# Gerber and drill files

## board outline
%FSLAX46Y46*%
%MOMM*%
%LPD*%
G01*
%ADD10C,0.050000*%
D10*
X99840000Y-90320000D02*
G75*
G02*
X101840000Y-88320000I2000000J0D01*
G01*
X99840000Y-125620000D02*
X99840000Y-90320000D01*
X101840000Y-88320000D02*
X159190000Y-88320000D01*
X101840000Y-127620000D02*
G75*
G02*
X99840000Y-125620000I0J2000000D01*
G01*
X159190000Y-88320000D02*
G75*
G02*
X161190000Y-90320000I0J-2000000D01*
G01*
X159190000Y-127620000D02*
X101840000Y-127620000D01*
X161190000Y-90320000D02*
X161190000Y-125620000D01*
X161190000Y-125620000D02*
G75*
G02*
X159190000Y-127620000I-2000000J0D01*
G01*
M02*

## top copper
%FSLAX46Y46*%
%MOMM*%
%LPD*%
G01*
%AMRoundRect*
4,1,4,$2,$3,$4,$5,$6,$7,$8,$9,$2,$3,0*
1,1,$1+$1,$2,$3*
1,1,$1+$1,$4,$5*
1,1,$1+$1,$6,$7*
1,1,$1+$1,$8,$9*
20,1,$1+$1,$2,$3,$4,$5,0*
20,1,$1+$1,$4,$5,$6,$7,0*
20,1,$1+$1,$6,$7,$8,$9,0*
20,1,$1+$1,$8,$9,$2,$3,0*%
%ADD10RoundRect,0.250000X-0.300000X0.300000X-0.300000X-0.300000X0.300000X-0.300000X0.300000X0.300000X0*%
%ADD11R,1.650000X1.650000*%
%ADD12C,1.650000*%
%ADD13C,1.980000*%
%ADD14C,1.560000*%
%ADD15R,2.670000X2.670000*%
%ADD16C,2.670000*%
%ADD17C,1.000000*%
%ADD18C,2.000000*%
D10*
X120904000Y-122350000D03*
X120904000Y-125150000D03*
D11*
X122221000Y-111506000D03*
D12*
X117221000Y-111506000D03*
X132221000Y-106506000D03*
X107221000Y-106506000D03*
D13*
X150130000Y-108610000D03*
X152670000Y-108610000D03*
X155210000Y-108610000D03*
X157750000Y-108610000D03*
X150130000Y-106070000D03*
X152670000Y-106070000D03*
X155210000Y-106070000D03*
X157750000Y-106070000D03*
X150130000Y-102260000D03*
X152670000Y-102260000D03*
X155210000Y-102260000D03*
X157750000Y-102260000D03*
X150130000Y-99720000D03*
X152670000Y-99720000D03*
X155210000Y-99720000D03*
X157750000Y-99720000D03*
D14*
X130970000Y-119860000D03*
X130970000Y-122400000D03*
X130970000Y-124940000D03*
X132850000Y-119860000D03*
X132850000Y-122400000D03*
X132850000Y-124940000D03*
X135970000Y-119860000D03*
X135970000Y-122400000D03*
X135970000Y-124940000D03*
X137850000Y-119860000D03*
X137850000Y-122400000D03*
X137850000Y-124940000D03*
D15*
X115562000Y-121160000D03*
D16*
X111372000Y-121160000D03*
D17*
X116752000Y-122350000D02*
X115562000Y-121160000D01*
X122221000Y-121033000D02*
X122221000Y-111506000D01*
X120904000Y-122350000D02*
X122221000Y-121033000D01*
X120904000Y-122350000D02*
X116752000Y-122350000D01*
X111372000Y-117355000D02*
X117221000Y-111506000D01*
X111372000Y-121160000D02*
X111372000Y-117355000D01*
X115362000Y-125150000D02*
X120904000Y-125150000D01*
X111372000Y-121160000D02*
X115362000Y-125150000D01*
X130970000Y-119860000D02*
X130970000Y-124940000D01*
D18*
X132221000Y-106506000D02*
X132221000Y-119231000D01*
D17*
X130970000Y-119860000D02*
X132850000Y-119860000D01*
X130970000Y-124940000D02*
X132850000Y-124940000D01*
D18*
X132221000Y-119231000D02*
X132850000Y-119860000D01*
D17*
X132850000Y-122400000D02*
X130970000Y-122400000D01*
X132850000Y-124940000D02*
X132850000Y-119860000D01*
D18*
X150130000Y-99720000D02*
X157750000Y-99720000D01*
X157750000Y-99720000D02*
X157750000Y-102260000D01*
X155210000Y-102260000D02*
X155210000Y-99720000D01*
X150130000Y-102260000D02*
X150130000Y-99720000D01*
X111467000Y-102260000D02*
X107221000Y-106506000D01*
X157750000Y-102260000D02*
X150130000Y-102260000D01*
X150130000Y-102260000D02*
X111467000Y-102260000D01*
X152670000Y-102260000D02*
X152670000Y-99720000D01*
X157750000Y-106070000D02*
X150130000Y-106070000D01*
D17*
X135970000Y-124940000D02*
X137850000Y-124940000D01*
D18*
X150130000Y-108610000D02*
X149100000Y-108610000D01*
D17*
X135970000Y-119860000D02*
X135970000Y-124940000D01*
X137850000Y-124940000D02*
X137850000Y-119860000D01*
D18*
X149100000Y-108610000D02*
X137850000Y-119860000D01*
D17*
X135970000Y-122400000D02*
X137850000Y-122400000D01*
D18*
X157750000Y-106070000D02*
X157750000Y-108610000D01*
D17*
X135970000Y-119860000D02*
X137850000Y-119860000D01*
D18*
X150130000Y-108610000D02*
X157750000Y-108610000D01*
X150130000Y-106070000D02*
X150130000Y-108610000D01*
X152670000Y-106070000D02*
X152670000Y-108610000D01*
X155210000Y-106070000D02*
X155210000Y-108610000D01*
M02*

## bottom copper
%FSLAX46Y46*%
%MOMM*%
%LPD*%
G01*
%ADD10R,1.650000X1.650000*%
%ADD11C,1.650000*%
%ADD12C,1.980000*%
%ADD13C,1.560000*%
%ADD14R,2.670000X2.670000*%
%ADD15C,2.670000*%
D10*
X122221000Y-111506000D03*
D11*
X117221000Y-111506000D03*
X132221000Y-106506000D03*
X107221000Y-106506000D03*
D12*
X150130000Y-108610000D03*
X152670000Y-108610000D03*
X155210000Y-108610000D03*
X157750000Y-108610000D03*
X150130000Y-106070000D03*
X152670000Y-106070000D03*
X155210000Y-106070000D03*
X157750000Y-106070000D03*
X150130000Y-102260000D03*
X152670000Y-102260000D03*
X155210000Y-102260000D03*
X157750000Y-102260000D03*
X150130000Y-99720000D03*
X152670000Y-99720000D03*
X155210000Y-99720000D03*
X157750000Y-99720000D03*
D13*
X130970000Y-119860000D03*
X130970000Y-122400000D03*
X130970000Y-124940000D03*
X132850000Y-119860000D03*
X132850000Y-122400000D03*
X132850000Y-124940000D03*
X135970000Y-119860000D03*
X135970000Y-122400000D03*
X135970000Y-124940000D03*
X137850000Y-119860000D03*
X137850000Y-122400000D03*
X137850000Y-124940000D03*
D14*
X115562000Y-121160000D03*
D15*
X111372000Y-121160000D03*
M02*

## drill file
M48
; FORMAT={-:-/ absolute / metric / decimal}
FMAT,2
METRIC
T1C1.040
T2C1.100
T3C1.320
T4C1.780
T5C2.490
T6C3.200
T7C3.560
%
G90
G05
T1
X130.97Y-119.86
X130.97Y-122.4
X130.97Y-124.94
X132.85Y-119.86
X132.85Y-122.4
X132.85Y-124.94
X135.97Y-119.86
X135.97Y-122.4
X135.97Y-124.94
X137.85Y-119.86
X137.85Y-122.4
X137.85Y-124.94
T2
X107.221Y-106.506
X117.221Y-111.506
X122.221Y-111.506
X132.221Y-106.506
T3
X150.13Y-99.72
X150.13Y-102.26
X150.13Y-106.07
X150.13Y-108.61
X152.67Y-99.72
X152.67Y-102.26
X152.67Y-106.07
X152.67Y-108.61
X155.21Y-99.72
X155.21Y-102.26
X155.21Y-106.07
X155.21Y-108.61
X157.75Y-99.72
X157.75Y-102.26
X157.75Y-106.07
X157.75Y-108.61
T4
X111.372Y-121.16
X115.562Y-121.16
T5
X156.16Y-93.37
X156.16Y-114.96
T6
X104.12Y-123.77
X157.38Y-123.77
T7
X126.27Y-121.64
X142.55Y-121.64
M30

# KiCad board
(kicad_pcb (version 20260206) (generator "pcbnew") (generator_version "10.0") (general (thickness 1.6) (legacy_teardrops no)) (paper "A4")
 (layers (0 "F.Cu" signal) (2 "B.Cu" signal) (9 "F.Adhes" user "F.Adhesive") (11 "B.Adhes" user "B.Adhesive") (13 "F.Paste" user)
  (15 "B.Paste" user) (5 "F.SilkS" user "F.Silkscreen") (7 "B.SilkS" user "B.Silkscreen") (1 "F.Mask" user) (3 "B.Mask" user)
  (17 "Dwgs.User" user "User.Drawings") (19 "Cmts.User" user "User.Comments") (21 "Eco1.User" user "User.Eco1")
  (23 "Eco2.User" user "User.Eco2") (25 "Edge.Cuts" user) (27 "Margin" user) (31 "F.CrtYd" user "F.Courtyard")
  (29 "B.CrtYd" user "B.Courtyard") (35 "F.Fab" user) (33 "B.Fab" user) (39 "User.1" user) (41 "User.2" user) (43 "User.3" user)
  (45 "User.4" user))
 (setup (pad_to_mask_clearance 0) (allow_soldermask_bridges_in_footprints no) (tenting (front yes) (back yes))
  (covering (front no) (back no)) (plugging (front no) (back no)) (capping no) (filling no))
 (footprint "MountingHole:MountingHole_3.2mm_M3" (layer "F.Cu") (at 104.12 123.77)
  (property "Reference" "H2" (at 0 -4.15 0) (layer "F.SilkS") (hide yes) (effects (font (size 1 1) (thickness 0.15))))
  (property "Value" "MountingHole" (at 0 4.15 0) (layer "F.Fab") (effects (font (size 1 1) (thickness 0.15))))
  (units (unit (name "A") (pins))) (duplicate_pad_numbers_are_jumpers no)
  (pad "" np_thru_hole circle (at 0 0) (size 3.2 3.2) (drill 3.2) (layers "*.Cu" "*.Mask")))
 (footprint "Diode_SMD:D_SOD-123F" (layer "F.Cu") (at 120.904 123.75 -90)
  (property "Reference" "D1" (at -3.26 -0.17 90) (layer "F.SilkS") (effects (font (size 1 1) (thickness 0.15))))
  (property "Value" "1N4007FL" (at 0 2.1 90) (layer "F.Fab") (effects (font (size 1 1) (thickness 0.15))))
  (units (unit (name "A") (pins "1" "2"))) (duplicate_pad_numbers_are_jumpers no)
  (pad "1" smd roundrect (at -1.4 0 270) (size 1.1 1.1) (layers "F.Cu" "F.Mask" "F.Paste") (roundrect_rratio 0.2272727273)
   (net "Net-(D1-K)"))
  (pad "2" smd roundrect (at 1.4 0 270) (size 1.1 1.1) (layers "F.Cu" "F.Mask" "F.Paste") (roundrect_rratio 0.2272727273) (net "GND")))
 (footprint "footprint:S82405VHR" (layer "F.Cu") (at 122.221 111.506 180)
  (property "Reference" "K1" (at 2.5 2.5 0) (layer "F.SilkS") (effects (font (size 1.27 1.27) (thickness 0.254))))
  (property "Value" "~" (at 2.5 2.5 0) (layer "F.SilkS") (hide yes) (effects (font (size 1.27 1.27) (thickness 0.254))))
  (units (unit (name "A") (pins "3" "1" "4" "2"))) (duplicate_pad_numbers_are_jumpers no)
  (pad "1" thru_hole rect (at 0 0 180) (size 1.65 1.65) (drill 1.1) (layers "*.Cu" "*.Mask") (remove_unused_layers no) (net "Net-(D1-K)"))
  (pad "2" thru_hole circle (at 5 0 180) (size 1.65 1.65) (drill 1.1) (layers "*.Cu" "*.Mask") (remove_unused_layers no) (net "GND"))
  (pad "3" thru_hole circle (at -10 5 180) (size 1.65 1.65) (drill 1.1) (layers "*.Cu" "*.Mask") (remove_unused_layers no)
   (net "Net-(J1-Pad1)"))
  (pad "4" thru_hole circle (at 15 5 180) (size 1.65 1.65) (drill 1.1) (layers "*.Cu" "*.Mask") (remove_unused_layers no)
   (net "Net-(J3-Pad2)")))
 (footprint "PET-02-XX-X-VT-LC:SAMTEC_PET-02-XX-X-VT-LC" (layer "F.Cu") (at 154.16 104.31 90)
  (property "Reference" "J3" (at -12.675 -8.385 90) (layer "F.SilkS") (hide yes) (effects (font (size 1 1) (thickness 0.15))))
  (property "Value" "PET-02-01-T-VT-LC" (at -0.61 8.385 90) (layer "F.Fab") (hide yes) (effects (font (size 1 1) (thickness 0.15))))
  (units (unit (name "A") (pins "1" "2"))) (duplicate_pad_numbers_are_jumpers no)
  (pad "" np_thru_hole circle (at -10.65 2 90) (size 2.49 2.49) (drill 2.49) (layers "*.Cu" "*.Mask"))
  (pad "" np_thru_hole circle (at 10.94 2 90) (size 2.49 2.49) (drill 2.49) (layers "*.Cu" "*.Mask"))
  (pad "1" thru_hole circle (at -4.3 -4.03 90) (size 1.98 1.98) (drill 1.32) (layers "*.Cu" "*.Mask") (remove_unused_layers no)
   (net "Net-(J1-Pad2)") (solder_mask_margin 0.102))
  (pad "1" thru_hole circle (at -4.3 -1.49 90) (size 1.98 1.98) (drill 1.32) (layers "*.Cu" "*.Mask") (remove_unused_layers no)
   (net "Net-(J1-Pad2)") (solder_mask_margin 0.102))
  (pad "1" thru_hole circle (at -4.3 1.05 90) (size 1.98 1.98) (drill 1.32) (layers "*.Cu" "*.Mask") (remove_unused_layers no)
   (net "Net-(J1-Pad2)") (solder_mask_margin 0.102))
  (pad "1" thru_hole circle (at -4.3 3.59 90) (size 1.98 1.98) (drill 1.32) (layers "*.Cu" "*.Mask") (remove_unused_layers no)
   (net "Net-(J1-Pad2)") (solder_mask_margin 0.102))
  (pad "1" thru_hole circle (at -1.76 -4.03 90) (size 1.98 1.98) (drill 1.32) (layers "*.Cu" "*.Mask") (remove_unused_layers no)
   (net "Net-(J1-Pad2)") (solder_mask_margin 0.102))
  (pad "1" thru_hole circle (at -1.76 -1.49 90) (size 1.98 1.98) (drill 1.32) (layers "*.Cu" "*.Mask") (remove_unused_layers no)
   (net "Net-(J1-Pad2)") (solder_mask_margin 0.102))
  (pad "1" thru_hole circle (at -1.76 1.05 90) (size 1.98 1.98) (drill 1.32) (layers "*.Cu" "*.Mask") (remove_unused_layers no)
   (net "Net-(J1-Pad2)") (solder_mask_margin 0.102))
  (pad "1" thru_hole circle (at -1.76 3.59 90) (size 1.98 1.98) (drill 1.32) (layers "*.Cu" "*.Mask") (remove_unused_layers no)
   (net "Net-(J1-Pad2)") (solder_mask_margin 0.102))
  (pad "2" thru_hole circle (at 2.05 -4.03 90) (size 1.98 1.98) (drill 1.32) (layers "*.Cu" "*.Mask") (remove_unused_layers no)
   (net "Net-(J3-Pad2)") (solder_mask_margin 0.102))
  (pad "2" thru_hole circle (at 2.05 -1.49 90) (size 1.98 1.98) (drill 1.32) (layers "*.Cu" "*.Mask") (remove_unused_layers no)
   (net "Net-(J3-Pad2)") (solder_mask_margin 0.102))
  (pad "2" thru_hole circle (at 2.05 1.05 90) (size 1.98 1.98) (drill 1.32) (layers "*.Cu" "*.Mask") (remove_unused_layers no)
   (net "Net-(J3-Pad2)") (solder_mask_margin 0.102))
  (pad "2" thru_hole circle (at 2.05 3.59 90) (size 1.98 1.98) (drill 1.32) (layers "*.Cu" "*.Mask") (remove_unused_layers no)
   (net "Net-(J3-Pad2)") (solder_mask_margin 0.102))
  (pad "2" thru_hole circle (at 4.59 -4.03 90) (size 1.98 1.98) (drill 1.32) (layers "*.Cu" "*.Mask") (remove_unused_layers no)
   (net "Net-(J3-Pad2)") (solder_mask_margin 0.102))
  (pad "2" thru_hole circle (at 4.59 -1.49 90) (size 1.98 1.98) (drill 1.32) (layers "*.Cu" "*.Mask") (remove_unused_layers no)
   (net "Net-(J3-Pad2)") (solder_mask_margin 0.102))
  (pad "2" thru_hole circle (at 4.59 1.05 90) (size 1.98 1.98) (drill 1.32) (layers "*.Cu" "*.Mask") (remove_unused_layers no)
   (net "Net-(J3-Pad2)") (solder_mask_margin 0.102))
  (pad "2" thru_hole circle (at 4.59 3.59 90) (size 1.98 1.98) (drill 1.32) (layers "*.Cu" "*.Mask") (remove_unused_layers no)
   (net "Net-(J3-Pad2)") (solder_mask_margin 0.102)))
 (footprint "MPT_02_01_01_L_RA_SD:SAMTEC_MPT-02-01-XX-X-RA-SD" (layer "F.Cu") (at 134.41 127.79)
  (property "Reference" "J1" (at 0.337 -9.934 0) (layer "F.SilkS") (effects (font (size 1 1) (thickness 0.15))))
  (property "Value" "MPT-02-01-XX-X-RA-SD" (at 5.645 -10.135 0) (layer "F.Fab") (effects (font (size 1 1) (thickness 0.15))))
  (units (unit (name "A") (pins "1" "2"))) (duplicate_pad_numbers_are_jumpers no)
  (pad "" np_thru_hole circle (at -8.14 -6.15) (size 3.56 3.56) (drill 3.56) (layers "*.Cu" "*.Mask"))
  (pad "" np_thru_hole circle (at 8.14 -6.15) (size 3.56 3.56) (drill 3.56) (layers "*.Cu" "*.Mask"))
  (pad "1" thru_hole circle (at -3.44 -7.93) (size 1.56 1.56) (drill 1.04) (layers "*.Cu" "*.Mask") (remove_unused_layers no)
   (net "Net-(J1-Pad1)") (solder_mask_margin 0.102))
  (pad "1" thru_hole circle (at -3.44 -5.39) (size 1.56 1.56) (drill 1.04) (layers "*.Cu" "*.Mask") (remove_unused_layers no)
   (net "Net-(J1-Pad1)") (solder_mask_margin 0.102))
  (pad "1" thru_hole circle (at -3.44 -2.85) (size 1.56 1.56) (drill 1.04) (layers "*.Cu" "*.Mask") (remove_unused_layers no)
   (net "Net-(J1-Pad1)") (solder_mask_margin 0.102))
  (pad "1" thru_hole circle (at -1.56 -7.93) (size 1.56 1.56) (drill 1.04) (layers "*.Cu" "*.Mask") (remove_unused_layers no)
   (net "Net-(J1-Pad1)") (solder_mask_margin 0.102))
  (pad "1" thru_hole circle (at -1.56 -5.39) (size 1.56 1.56) (drill 1.04) (layers "*.Cu" "*.Mask") (remove_unused_layers no)
   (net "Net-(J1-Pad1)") (solder_mask_margin 0.102))
  (pad "1" thru_hole circle (at -1.56 -2.85) (size 1.56 1.56) (drill 1.04) (layers "*.Cu" "*.Mask") (remove_unused_layers no)
   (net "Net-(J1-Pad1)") (solder_mask_margin 0.102))
  (pad "2" thru_hole circle (at 1.56 -7.93) (size 1.56 1.56) (drill 1.04) (layers "*.Cu" "*.Mask") (remove_unused_layers no)
   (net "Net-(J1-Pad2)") (solder_mask_margin 0.102))
  (pad "2" thru_hole circle (at 1.56 -5.39) (size 1.56 1.56) (drill 1.04) (layers "*.Cu" "*.Mask") (remove_unused_layers no)
   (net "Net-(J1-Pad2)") (solder_mask_margin 0.102))
  (pad "2" thru_hole circle (at 1.56 -2.85) (size 1.56 1.56) (drill 1.04) (layers "*.Cu" "*.Mask") (remove_unused_layers no)
   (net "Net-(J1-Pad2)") (solder_mask_margin 0.102))
  (pad "2" thru_hole circle (at 3.44 -7.93) (size 1.56 1.56) (drill 1.04) (layers "*.Cu" "*.Mask") (remove_unused_layers no)
   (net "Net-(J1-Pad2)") (solder_mask_margin 0.102))
  (pad "2" thru_hole circle (at 3.44 -5.39) (size 1.56 1.56) (drill 1.04) (layers "*.Cu" "*.Mask") (remove_unused_layers no)
   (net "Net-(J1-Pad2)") (solder_mask_margin 0.102))
  (pad "2" thru_hole circle (at 3.44 -2.85) (size 1.56 1.56) (drill 1.04) (layers "*.Cu" "*.Mask") (remove_unused_layers no)
   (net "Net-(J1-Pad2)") (solder_mask_margin 0.102)))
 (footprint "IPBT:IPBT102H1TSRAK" (layer "F.Cu") (at 115.562 121.16 180)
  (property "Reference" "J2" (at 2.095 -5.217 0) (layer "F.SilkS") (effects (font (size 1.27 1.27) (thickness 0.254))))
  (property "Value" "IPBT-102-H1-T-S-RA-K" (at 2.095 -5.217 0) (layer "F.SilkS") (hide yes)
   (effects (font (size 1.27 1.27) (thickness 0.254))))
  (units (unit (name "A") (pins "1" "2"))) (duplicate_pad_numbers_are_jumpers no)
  (pad "1" thru_hole rect (at 0 0 180) (size 2.67 2.67) (drill 1.78) (layers "*.Cu" "*.Mask") (remove_unused_layers no) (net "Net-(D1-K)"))
  (pad "2" thru_hole circle (at 4.19 0 180) (size 2.67 2.67) (drill 1.78) (layers "*.Cu" "*.Mask") (remove_unused_layers no) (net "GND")))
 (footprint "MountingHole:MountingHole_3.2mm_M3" (layer "F.Cu") (at 157.38 123.77)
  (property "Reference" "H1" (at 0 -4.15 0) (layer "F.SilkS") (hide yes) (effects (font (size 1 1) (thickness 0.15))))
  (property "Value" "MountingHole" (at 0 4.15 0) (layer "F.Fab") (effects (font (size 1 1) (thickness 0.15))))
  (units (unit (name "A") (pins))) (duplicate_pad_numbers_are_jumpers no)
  (pad "" np_thru_hole circle (at 0 0) (size 3.2 3.2) (drill 3.2) (layers "*.Cu" "*.Mask")))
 (gr_arc (start 99.84 90.32) (mid 100.425786 88.905786) (end 101.84 88.32) (stroke (width 0.05) (type default)) (layer "Edge.Cuts"))
 (gr_line (start 99.84 125.62) (end 99.84 90.32) (stroke (width 0.05) (type default)) (layer "Edge.Cuts"))
 (gr_line (start 101.84 88.32) (end 159.19 88.32) (stroke (width 0.05) (type default)) (layer "Edge.Cuts"))
 (gr_arc (start 101.84 127.62) (mid 100.425786 127.034214) (end 99.84 125.62) (stroke (width 0.05) (type default)) (layer "Edge.Cuts"))
 (gr_arc (start 159.19 88.32) (mid 160.604214 88.905786) (end 161.19 90.32) (stroke (width 0.05) (type default)) (layer "Edge.Cuts"))
 (gr_line (start 159.19 127.62) (end 101.84 127.62) (stroke (width 0.05) (type default)) (layer "Edge.Cuts"))
 (gr_line (start 161.19 90.32) (end 161.19 125.62) (stroke (width 0.05) (type default)) (layer "Edge.Cuts"))
 (gr_arc (start 161.19 125.62) (mid 160.604214 127.034214) (end 159.19 127.62) (stroke (width 0.05) (type default)) (layer "Edge.Cuts"))
 (segment (start 116.752 122.35) (end 115.562 121.16) (width 1) (layer "F.Cu") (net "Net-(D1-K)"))
 (segment (start 122.221 121.033) (end 122.221 111.506) (width 1) (layer "F.Cu") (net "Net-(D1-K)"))
 (segment (start 120.904 122.35) (end 122.221 121.033) (width 1) (layer "F.Cu") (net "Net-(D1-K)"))
 (segment (start 120.904 122.35) (end 116.752 122.35) (width 1) (layer "F.Cu") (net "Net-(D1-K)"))
 (segment (start 111.372 117.355) (end 117.221 111.506) (width 1) (layer "F.Cu") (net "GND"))
 (segment (start 111.372 121.16) (end 111.372 117.355) (width 1) (layer "F.Cu") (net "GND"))
 (segment (start 115.362 125.15) (end 120.904 125.15) (width 1) (layer "F.Cu") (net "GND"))
 (segment (start 111.372 121.16) (end 115.362 125.15) (width 1) (layer "F.Cu") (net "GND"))
 (segment (start 130.97 119.86) (end 130.97 124.94) (width 1) (layer "F.Cu") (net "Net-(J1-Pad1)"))
 (segment (start 132.221 106.506) (end 132.221 119.231) (width 2) (layer "F.Cu") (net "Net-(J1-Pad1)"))
 (segment (start 130.97 119.86) (end 132.85 119.86) (width 1) (layer "F.Cu") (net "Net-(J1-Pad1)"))
 (segment (start 130.97 124.94) (end 132.85 124.94) (width 1) (layer "F.Cu") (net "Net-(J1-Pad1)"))
 (segment (start 132.221 119.231) (end 132.85 119.86) (width 2) (layer "F.Cu") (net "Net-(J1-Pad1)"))
 (segment (start 132.85 122.4) (end 130.97 122.4) (width 1) (layer "F.Cu") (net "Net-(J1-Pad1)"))
 (segment (start 132.85 124.94) (end 132.85 119.86) (width 1) (layer "F.Cu") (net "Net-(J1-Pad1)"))
 (segment (start 150.13 99.72) (end 157.75 99.72) (width 2) (layer "F.Cu") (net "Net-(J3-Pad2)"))
 (segment (start 157.75 99.72) (end 157.75 102.26) (width 2) (layer "F.Cu") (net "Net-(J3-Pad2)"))
 (segment (start 155.21 102.26) (end 155.21 99.72) (width 2) (layer "F.Cu") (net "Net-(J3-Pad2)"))
 (segment (start 150.13 102.26) (end 150.13 99.72) (width 2) (layer "F.Cu") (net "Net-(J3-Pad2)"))
 (segment (start 111.467 102.26) (end 107.221 106.506) (width 2) (layer "F.Cu") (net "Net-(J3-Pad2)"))
 (segment (start 157.75 102.26) (end 150.13 102.26) (width 2) (layer "F.Cu") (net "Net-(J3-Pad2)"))
 (segment (start 150.13 102.26) (end 111.467 102.26) (width 2) (layer "F.Cu") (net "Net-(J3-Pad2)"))
 (segment (start 152.67 102.26) (end 152.67 99.72) (width 2) (layer "F.Cu") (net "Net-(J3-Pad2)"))
 (segment (start 157.75 106.07) (end 150.13 106.07) (width 2) (layer "F.Cu") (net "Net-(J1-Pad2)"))
 (segment (start 135.97 124.94) (end 137.85 124.94) (width 1) (layer "F.Cu") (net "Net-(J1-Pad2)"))
 (segment (start 150.13 108.61) (end 149.1 108.61) (width 2) (layer "F.Cu") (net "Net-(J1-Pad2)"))
 (segment (start 135.97 119.86) (end 135.97 124.94) (width 1) (layer "F.Cu") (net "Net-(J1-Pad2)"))
 (segment (start 137.85 124.94) (end 137.85 119.86) (width 1) (layer "F.Cu") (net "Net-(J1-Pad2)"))
 (segment (start 149.1 108.61) (end 137.85 119.86) (width 2) (layer "F.Cu") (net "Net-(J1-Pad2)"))
 (segment (start 135.97 122.4) (end 137.85 122.4) (width 1) (layer "F.Cu") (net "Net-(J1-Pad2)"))
 (segment (start 157.75 106.07) (end 157.75 108.61) (width 2) (layer "F.Cu") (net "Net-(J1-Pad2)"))
 (segment (start 135.97 119.86) (end 137.85 119.86) (width 1) (layer "F.Cu") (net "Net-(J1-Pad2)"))
 (segment (start 150.13 108.61) (end 157.75 108.61) (width 2) (layer "F.Cu") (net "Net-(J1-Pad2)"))
 (segment (start 150.13 106.07) (end 150.13 108.61) (width 2) (layer "F.Cu") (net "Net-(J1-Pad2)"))
 (segment (start 152.67 106.07) (end 152.67 108.61) (width 2) (layer "F.Cu") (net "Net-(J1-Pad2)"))
 (segment (start 155.21 106.07) (end 155.21 108.61) (width 2) (layer "F.Cu") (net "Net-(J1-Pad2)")))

